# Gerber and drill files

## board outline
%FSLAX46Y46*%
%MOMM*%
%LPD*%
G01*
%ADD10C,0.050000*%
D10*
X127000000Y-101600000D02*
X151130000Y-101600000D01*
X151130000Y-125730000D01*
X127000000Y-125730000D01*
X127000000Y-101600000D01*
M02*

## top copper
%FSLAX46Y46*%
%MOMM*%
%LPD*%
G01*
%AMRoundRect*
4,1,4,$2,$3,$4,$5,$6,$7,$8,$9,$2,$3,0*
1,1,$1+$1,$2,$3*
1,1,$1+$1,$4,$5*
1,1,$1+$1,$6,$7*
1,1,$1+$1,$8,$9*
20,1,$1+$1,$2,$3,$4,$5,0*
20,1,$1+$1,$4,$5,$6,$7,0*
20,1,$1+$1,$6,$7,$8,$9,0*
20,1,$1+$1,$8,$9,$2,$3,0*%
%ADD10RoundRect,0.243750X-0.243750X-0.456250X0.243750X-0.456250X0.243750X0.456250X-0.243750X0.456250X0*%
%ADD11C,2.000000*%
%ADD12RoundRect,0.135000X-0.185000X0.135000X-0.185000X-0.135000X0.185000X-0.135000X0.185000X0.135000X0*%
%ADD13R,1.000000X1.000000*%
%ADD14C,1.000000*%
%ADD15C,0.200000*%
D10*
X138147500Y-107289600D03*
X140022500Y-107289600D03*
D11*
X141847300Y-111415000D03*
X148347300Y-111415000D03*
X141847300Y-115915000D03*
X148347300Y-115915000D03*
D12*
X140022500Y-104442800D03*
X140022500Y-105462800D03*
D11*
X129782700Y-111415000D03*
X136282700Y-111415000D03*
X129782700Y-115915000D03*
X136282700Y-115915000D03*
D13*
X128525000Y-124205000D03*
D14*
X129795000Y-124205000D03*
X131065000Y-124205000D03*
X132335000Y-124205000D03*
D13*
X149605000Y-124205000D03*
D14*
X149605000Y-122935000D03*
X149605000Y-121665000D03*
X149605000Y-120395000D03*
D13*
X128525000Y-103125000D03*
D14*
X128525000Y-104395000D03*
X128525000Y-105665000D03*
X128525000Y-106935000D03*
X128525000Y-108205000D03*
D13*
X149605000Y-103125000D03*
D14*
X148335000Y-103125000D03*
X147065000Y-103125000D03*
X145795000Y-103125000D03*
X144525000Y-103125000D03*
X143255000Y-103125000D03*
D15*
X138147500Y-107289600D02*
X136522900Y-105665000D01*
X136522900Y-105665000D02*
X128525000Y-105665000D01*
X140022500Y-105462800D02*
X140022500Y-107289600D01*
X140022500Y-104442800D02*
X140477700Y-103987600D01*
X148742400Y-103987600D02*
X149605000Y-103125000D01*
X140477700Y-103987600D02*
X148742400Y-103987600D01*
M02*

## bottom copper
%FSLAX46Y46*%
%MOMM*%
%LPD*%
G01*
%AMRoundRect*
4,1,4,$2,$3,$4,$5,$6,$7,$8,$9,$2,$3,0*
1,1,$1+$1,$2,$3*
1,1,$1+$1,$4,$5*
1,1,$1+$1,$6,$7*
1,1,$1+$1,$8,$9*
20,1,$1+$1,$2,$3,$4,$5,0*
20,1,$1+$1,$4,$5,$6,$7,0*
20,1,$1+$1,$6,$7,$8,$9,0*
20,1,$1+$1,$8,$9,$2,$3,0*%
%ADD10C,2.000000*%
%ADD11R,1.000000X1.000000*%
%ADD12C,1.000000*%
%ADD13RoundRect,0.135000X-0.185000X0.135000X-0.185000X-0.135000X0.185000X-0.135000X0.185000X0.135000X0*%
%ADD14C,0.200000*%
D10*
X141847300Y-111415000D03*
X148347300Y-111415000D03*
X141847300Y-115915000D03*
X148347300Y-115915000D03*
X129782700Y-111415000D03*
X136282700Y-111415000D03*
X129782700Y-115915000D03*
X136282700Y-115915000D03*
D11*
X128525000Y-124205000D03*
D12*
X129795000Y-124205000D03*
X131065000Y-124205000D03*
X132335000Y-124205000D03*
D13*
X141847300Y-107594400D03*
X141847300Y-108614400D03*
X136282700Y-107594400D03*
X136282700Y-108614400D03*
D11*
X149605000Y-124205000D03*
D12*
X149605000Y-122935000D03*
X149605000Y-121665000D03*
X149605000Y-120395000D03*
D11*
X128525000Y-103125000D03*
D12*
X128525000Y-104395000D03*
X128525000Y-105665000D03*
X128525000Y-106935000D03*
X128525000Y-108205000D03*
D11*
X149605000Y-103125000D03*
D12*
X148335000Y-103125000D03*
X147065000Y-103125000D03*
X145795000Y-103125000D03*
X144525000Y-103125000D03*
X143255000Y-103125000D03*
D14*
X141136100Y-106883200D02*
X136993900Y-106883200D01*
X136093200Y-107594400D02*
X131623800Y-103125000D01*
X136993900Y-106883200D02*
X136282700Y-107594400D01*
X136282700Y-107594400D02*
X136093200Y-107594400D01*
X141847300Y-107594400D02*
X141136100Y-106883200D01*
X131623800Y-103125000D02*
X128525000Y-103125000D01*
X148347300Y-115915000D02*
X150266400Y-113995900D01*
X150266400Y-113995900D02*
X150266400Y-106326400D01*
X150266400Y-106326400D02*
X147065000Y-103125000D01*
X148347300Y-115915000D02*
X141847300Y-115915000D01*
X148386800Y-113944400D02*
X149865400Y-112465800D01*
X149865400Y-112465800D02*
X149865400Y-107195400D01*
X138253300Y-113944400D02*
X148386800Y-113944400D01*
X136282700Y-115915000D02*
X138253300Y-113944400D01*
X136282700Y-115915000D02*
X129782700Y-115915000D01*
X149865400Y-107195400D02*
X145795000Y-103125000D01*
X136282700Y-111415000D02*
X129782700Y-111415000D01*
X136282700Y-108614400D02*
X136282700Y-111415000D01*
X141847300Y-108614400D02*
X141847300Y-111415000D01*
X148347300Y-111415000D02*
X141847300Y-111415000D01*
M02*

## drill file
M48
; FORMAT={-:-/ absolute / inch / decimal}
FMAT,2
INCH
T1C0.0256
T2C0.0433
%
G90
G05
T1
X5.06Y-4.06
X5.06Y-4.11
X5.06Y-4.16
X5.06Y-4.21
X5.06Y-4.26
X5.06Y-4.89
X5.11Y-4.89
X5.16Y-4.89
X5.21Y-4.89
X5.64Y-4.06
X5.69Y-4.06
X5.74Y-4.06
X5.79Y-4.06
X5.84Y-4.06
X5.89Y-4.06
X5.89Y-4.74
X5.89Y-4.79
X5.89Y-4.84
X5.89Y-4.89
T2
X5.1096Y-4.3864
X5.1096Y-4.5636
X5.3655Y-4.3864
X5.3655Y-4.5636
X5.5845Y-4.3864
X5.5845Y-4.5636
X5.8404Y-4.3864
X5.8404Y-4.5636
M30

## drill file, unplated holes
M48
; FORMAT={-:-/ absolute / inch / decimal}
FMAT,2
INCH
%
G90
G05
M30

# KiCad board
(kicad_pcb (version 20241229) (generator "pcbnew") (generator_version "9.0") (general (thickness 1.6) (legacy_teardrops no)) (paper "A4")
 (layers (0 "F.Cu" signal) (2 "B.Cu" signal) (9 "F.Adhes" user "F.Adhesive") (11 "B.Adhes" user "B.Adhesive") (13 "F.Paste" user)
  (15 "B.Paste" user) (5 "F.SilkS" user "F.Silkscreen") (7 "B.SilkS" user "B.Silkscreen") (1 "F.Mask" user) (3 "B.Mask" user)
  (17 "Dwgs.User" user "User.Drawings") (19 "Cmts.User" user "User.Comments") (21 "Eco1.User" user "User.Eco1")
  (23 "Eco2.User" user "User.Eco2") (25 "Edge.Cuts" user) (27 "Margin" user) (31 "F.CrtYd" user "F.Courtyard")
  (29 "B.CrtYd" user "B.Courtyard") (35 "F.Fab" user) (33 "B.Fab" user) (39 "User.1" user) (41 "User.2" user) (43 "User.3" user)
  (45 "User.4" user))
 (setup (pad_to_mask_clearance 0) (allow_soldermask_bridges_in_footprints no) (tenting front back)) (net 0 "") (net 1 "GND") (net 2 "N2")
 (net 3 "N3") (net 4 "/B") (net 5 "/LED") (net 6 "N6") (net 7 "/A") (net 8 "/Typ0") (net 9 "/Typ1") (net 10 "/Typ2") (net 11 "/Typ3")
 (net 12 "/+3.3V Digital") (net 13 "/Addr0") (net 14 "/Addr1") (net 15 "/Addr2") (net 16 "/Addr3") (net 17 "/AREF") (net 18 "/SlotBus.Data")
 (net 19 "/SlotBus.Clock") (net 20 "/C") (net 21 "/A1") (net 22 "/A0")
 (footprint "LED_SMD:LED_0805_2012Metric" (layer "F.Cu") (at 139.085 107.2896)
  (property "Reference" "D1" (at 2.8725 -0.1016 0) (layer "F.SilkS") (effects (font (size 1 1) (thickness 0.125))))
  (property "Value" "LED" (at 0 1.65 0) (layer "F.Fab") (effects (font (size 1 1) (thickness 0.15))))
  (pad "1" smd roundrect (at -0.9375 0) (size 0.975 1.4) (layers "F.Cu" "F.Mask" "F.Paste") (roundrect_rratio 0.25) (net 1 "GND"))
  (pad "2" smd roundrect (at 0.9375 0) (size 0.975 1.4) (layers "F.Cu" "F.Mask" "F.Paste") (roundrect_rratio 0.25) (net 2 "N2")))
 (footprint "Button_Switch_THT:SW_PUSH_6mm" (layer "F.Cu") (at 141.8473 111.415)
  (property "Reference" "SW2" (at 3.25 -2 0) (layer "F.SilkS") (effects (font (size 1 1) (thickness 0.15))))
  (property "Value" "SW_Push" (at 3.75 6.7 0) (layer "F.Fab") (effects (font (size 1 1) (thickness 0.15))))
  (pad "1" thru_hole circle (at 0 0 90) (size 2 2) (drill 1.1) (layers "*.Cu" "*.Mask") (remove_unused_layers no) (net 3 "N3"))
  (pad "1" thru_hole circle (at 6.5 0 90) (size 2 2) (drill 1.1) (layers "*.Cu" "*.Mask") (remove_unused_layers no) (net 3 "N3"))
  (pad "2" thru_hole circle (at 0 4.5 90) (size 2 2) (drill 1.1) (layers "*.Cu" "*.Mask") (remove_unused_layers no) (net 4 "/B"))
  (pad "2" thru_hole circle (at 6.5 4.5 90) (size 2 2) (drill 1.1) (layers "*.Cu" "*.Mask") (remove_unused_layers no) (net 4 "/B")))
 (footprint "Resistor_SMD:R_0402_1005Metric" (layer "F.Cu") (at 140.0225 104.9528 -90)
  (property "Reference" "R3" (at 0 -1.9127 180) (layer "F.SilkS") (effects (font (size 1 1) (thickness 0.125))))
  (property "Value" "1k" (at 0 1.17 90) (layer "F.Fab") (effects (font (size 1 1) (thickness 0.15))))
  (pad "1" smd roundrect (at -0.51 0 270) (size 0.54 0.64) (layers "F.Cu" "F.Mask" "F.Paste") (roundrect_rratio 0.25) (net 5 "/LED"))
  (pad "2" smd roundrect (at 0.51 0 270) (size 0.54 0.64) (layers "F.Cu" "F.Mask" "F.Paste") (roundrect_rratio 0.25) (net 2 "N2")))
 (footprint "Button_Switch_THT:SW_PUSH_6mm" (layer "F.Cu") (at 129.7827 111.415)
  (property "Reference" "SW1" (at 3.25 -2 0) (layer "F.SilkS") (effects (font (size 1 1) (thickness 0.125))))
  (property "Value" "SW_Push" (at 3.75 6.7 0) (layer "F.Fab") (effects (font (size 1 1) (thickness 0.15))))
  (pad "1" thru_hole circle (at 0 0 90) (size 2 2) (drill 1.1) (layers "*.Cu" "*.Mask") (remove_unused_layers no) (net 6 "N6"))
  (pad "1" thru_hole circle (at 6.5 0 90) (size 2 2) (drill 1.1) (layers "*.Cu" "*.Mask") (remove_unused_layers no) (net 6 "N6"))
  (pad "2" thru_hole circle (at 0 4.5 90) (size 2 2) (drill 1.1) (layers "*.Cu" "*.Mask") (remove_unused_layers no) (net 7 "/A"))
  (pad "2" thru_hole circle (at 6.5 4.5 90) (size 2 2) (drill 1.1) (layers "*.Cu" "*.Mask") (remove_unused_layers no) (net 7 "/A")))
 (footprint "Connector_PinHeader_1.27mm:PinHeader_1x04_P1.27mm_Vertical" (layer "B.Cu") (at 128.525 124.205 -90)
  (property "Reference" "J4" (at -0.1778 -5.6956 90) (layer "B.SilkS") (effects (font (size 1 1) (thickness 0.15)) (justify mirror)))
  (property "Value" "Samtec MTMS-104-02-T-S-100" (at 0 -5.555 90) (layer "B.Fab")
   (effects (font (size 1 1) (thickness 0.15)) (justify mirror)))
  (pad "1" thru_hole rect (at 0 0 270) (size 1 1) (drill 0.65) (layers "*.Cu" "*.Mask") (remove_unused_layers no) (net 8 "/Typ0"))
  (pad "2" thru_hole circle (at 0 -1.27 270) (size 1 1) (drill 0.65) (layers "*.Cu" "*.Mask") (remove_unused_layers no) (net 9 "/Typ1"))
  (pad "3" thru_hole circle (at 0 -2.54 270) (size 1 1) (drill 0.65) (layers "*.Cu" "*.Mask") (remove_unused_layers no) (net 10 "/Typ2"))
  (pad "4" thru_hole circle (at 0 -3.81 270) (size 1 1) (drill 0.65) (layers "*.Cu" "*.Mask") (remove_unused_layers no) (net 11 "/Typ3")))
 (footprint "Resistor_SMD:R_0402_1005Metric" (layer "B.Cu") (at 141.8473 108.1044 -90)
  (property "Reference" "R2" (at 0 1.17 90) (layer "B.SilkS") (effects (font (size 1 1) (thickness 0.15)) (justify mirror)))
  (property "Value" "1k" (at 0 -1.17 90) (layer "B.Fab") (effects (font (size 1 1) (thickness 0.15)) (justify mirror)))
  (pad "1" smd roundrect (at -0.51 0 270) (size 0.54 0.64) (layers "B.Cu" "B.Mask" "B.Paste") (roundrect_rratio 0.25)
   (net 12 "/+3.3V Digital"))
  (pad "2" smd roundrect (at 0.51 0 270) (size 0.54 0.64) (layers "B.Cu" "B.Mask" "B.Paste") (roundrect_rratio 0.25) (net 3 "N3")))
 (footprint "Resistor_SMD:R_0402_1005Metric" (layer "B.Cu") (at 136.2827 108.1044 -90)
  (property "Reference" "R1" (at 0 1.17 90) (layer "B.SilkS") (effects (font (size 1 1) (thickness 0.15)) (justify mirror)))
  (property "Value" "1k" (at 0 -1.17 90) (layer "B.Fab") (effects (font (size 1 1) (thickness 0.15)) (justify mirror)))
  (pad "1" smd roundrect (at -0.51 0 270) (size 0.54 0.64) (layers "B.Cu" "B.Mask" "B.Paste") (roundrect_rratio 0.25)
   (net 12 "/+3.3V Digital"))
  (pad "2" smd roundrect (at 0.51 0 270) (size 0.54 0.64) (layers "B.Cu" "B.Mask" "B.Paste") (roundrect_rratio 0.25) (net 6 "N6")))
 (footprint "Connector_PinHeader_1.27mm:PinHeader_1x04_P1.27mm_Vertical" (layer "B.Cu") (at 149.605 124.205)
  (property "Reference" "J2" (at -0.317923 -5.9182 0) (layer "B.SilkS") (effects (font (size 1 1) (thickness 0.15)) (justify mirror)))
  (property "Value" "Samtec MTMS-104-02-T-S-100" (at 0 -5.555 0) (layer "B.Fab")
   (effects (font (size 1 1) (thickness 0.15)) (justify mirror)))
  (pad "1" thru_hole rect (at 0 0) (size 1 1) (drill 0.65) (layers "*.Cu" "*.Mask") (remove_unused_layers no) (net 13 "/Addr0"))
  (pad "2" thru_hole circle (at 0 -1.27) (size 1 1) (drill 0.65) (layers "*.Cu" "*.Mask") (remove_unused_layers no) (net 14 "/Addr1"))
  (pad "3" thru_hole circle (at 0 -2.54) (size 1 1) (drill 0.65) (layers "*.Cu" "*.Mask") (remove_unused_layers no) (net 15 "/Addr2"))
  (pad "4" thru_hole circle (at 0 -3.81) (size 1 1) (drill 0.65) (layers "*.Cu" "*.Mask") (remove_unused_layers no) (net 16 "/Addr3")))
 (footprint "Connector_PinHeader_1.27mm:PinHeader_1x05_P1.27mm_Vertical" (layer "B.Cu") (at 128.525 103.125 180)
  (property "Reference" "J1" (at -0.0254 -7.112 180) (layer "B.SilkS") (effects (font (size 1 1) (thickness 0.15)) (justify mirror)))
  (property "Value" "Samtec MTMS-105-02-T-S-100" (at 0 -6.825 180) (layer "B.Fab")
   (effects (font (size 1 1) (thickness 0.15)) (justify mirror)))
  (pad "1" thru_hole rect (at 0 0 180) (size 1 1) (drill 0.65) (layers "*.Cu" "*.Mask") (remove_unused_layers no) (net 12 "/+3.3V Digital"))
  (pad "2" thru_hole circle (at 0 -1.27 180) (size 1 1) (drill 0.65) (layers "*.Cu" "*.Mask") (remove_unused_layers no) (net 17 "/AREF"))
  (pad "3" thru_hole circle (at 0 -2.54 180) (size 1 1) (drill 0.65) (layers "*.Cu" "*.Mask") (remove_unused_layers no) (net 1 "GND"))
  (pad "4" thru_hole circle (at 0 -3.81 180) (size 1 1) (drill 0.65) (layers "*.Cu" "*.Mask") (remove_unused_layers no)
   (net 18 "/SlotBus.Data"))
  (pad "5" thru_hole circle (at 0 -5.08 180) (size 1 1) (drill 0.65) (layers "*.Cu" "*.Mask") (remove_unused_layers no)
   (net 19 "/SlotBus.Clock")))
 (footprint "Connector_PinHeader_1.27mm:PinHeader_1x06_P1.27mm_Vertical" (layer "B.Cu") (at 149.605 103.125 90)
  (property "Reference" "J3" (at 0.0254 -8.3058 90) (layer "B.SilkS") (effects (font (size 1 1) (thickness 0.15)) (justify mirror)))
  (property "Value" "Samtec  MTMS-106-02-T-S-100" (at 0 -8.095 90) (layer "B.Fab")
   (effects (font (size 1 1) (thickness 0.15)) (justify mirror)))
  (pad "1" thru_hole rect (at 0 0 90) (size 1 1) (drill 0.65) (layers "*.Cu" "*.Mask") (remove_unused_layers no) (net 5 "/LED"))
  (pad "2" thru_hole circle (at 0 -1.27 90) (size 1 1) (drill 0.65) (layers "*.Cu" "*.Mask") (remove_unused_layers no) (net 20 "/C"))
  (pad "3" thru_hole circle (at 0 -2.54 90) (size 1 1) (drill 0.65) (layers "*.Cu" "*.Mask") (remove_unused_layers no) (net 4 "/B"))
  (pad "4" thru_hole circle (at 0 -3.81 90) (size 1 1) (drill 0.65) (layers "*.Cu" "*.Mask") (remove_unused_layers no) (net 7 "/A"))
  (pad "5" thru_hole circle (at 0 -5.08 90) (size 1 1) (drill 0.65) (layers "*.Cu" "*.Mask") (remove_unused_layers no) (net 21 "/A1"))
  (pad "6" thru_hole circle (at 0 -6.35 90) (size 1 1) (drill 0.65) (layers "*.Cu" "*.Mask") (remove_unused_layers no) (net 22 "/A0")))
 (gr_rect (start 127 101.6) (end 151.13 125.73) (stroke (width 0.05) (type solid)) (fill no) (layer "Edge.Cuts"))
 (segment (start 138.1475 107.2896) (end 136.5229 105.665) (width 0.2) (layer "F.Cu") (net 1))
 (segment (start 136.5229 105.665) (end 128.525 105.665) (width 0.2) (layer "F.Cu") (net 1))
 (segment (start 140.0225 105.4628) (end 140.0225 107.2896) (width 0.2) (layer "F.Cu") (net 2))
 (segment (start 141.1361 106.8832) (end 136.9939 106.8832) (width 0.2) (layer "B.Cu") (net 12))
 (segment (start 136.0932 107.5944) (end 131.6238 103.125) (width 0.2) (layer "B.Cu") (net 12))
 (segment (start 136.9939 106.8832) (end 136.2827 107.5944) (width 0.2) (layer "B.Cu") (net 12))
 (segment (start 136.2827 107.5944) (end 136.0932 107.5944) (width 0.2) (layer "B.Cu") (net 12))
 (segment (start 141.8473 107.5944) (end 141.1361 106.8832) (width 0.2) (layer "B.Cu") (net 12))
 (segment (start 131.6238 103.125) (end 128.525 103.125) (width 0.2) (layer "B.Cu") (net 12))
 (segment (start 148.3473 115.915) (end 150.2664 113.9959) (width 0.2) (layer "B.Cu") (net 4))
 (segment (start 150.2664 113.9959) (end 150.2664 106.3264) (width 0.2) (layer "B.Cu") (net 4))
 (segment (start 150.2664 106.3264) (end 147.065 103.125) (width 0.2) (layer "B.Cu") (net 4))
 (segment (start 148.3473 115.915) (end 141.8473 115.915) (width 0.2) (layer "B.Cu") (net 4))
 (segment (start 140.0225 104.4428) (end 140.4777 103.9876) (width 0.2) (layer "F.Cu") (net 5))
 (segment (start 148.7424 103.9876) (end 149.605 103.125) (width 0.2) (layer "F.Cu") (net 5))
 (segment (start 140.4777 103.9876) (end 148.7424 103.9876) (width 0.2) (layer "F.Cu") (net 5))
 (segment (start 148.3868 113.9444) (end 149.8654 112.4658) (width 0.2) (layer "B.Cu") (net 7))
 (segment (start 149.8654 112.4658) (end 149.8654 107.1954) (width 0.2) (layer "B.Cu") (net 7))
 (segment (start 138.2533 113.9444) (end 148.3868 113.9444) (width 0.2) (layer "B.Cu") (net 7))
 (segment (start 136.2827 115.915) (end 138.2533 113.9444) (width 0.2) (layer "B.Cu") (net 7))
 (segment (start 136.2827 115.915) (end 129.7827 115.915) (width 0.2) (layer "B.Cu") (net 7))
 (segment (start 149.8654 107.1954) (end 145.795 103.125) (width 0.2) (layer "B.Cu") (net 7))
 (segment (start 136.2827 111.415) (end 129.7827 111.415) (width 0.2) (layer "B.Cu") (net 6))
 (segment (start 136.2827 108.6144) (end 136.2827 111.415) (width 0.2) (layer "B.Cu") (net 6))
 (segment (start 141.8473 108.6144) (end 141.8473 111.415) (width 0.2) (layer "B.Cu") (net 3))
 (segment (start 148.3473 111.415) (end 141.8473 111.415) (width 0.2) (layer "B.Cu") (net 3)))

